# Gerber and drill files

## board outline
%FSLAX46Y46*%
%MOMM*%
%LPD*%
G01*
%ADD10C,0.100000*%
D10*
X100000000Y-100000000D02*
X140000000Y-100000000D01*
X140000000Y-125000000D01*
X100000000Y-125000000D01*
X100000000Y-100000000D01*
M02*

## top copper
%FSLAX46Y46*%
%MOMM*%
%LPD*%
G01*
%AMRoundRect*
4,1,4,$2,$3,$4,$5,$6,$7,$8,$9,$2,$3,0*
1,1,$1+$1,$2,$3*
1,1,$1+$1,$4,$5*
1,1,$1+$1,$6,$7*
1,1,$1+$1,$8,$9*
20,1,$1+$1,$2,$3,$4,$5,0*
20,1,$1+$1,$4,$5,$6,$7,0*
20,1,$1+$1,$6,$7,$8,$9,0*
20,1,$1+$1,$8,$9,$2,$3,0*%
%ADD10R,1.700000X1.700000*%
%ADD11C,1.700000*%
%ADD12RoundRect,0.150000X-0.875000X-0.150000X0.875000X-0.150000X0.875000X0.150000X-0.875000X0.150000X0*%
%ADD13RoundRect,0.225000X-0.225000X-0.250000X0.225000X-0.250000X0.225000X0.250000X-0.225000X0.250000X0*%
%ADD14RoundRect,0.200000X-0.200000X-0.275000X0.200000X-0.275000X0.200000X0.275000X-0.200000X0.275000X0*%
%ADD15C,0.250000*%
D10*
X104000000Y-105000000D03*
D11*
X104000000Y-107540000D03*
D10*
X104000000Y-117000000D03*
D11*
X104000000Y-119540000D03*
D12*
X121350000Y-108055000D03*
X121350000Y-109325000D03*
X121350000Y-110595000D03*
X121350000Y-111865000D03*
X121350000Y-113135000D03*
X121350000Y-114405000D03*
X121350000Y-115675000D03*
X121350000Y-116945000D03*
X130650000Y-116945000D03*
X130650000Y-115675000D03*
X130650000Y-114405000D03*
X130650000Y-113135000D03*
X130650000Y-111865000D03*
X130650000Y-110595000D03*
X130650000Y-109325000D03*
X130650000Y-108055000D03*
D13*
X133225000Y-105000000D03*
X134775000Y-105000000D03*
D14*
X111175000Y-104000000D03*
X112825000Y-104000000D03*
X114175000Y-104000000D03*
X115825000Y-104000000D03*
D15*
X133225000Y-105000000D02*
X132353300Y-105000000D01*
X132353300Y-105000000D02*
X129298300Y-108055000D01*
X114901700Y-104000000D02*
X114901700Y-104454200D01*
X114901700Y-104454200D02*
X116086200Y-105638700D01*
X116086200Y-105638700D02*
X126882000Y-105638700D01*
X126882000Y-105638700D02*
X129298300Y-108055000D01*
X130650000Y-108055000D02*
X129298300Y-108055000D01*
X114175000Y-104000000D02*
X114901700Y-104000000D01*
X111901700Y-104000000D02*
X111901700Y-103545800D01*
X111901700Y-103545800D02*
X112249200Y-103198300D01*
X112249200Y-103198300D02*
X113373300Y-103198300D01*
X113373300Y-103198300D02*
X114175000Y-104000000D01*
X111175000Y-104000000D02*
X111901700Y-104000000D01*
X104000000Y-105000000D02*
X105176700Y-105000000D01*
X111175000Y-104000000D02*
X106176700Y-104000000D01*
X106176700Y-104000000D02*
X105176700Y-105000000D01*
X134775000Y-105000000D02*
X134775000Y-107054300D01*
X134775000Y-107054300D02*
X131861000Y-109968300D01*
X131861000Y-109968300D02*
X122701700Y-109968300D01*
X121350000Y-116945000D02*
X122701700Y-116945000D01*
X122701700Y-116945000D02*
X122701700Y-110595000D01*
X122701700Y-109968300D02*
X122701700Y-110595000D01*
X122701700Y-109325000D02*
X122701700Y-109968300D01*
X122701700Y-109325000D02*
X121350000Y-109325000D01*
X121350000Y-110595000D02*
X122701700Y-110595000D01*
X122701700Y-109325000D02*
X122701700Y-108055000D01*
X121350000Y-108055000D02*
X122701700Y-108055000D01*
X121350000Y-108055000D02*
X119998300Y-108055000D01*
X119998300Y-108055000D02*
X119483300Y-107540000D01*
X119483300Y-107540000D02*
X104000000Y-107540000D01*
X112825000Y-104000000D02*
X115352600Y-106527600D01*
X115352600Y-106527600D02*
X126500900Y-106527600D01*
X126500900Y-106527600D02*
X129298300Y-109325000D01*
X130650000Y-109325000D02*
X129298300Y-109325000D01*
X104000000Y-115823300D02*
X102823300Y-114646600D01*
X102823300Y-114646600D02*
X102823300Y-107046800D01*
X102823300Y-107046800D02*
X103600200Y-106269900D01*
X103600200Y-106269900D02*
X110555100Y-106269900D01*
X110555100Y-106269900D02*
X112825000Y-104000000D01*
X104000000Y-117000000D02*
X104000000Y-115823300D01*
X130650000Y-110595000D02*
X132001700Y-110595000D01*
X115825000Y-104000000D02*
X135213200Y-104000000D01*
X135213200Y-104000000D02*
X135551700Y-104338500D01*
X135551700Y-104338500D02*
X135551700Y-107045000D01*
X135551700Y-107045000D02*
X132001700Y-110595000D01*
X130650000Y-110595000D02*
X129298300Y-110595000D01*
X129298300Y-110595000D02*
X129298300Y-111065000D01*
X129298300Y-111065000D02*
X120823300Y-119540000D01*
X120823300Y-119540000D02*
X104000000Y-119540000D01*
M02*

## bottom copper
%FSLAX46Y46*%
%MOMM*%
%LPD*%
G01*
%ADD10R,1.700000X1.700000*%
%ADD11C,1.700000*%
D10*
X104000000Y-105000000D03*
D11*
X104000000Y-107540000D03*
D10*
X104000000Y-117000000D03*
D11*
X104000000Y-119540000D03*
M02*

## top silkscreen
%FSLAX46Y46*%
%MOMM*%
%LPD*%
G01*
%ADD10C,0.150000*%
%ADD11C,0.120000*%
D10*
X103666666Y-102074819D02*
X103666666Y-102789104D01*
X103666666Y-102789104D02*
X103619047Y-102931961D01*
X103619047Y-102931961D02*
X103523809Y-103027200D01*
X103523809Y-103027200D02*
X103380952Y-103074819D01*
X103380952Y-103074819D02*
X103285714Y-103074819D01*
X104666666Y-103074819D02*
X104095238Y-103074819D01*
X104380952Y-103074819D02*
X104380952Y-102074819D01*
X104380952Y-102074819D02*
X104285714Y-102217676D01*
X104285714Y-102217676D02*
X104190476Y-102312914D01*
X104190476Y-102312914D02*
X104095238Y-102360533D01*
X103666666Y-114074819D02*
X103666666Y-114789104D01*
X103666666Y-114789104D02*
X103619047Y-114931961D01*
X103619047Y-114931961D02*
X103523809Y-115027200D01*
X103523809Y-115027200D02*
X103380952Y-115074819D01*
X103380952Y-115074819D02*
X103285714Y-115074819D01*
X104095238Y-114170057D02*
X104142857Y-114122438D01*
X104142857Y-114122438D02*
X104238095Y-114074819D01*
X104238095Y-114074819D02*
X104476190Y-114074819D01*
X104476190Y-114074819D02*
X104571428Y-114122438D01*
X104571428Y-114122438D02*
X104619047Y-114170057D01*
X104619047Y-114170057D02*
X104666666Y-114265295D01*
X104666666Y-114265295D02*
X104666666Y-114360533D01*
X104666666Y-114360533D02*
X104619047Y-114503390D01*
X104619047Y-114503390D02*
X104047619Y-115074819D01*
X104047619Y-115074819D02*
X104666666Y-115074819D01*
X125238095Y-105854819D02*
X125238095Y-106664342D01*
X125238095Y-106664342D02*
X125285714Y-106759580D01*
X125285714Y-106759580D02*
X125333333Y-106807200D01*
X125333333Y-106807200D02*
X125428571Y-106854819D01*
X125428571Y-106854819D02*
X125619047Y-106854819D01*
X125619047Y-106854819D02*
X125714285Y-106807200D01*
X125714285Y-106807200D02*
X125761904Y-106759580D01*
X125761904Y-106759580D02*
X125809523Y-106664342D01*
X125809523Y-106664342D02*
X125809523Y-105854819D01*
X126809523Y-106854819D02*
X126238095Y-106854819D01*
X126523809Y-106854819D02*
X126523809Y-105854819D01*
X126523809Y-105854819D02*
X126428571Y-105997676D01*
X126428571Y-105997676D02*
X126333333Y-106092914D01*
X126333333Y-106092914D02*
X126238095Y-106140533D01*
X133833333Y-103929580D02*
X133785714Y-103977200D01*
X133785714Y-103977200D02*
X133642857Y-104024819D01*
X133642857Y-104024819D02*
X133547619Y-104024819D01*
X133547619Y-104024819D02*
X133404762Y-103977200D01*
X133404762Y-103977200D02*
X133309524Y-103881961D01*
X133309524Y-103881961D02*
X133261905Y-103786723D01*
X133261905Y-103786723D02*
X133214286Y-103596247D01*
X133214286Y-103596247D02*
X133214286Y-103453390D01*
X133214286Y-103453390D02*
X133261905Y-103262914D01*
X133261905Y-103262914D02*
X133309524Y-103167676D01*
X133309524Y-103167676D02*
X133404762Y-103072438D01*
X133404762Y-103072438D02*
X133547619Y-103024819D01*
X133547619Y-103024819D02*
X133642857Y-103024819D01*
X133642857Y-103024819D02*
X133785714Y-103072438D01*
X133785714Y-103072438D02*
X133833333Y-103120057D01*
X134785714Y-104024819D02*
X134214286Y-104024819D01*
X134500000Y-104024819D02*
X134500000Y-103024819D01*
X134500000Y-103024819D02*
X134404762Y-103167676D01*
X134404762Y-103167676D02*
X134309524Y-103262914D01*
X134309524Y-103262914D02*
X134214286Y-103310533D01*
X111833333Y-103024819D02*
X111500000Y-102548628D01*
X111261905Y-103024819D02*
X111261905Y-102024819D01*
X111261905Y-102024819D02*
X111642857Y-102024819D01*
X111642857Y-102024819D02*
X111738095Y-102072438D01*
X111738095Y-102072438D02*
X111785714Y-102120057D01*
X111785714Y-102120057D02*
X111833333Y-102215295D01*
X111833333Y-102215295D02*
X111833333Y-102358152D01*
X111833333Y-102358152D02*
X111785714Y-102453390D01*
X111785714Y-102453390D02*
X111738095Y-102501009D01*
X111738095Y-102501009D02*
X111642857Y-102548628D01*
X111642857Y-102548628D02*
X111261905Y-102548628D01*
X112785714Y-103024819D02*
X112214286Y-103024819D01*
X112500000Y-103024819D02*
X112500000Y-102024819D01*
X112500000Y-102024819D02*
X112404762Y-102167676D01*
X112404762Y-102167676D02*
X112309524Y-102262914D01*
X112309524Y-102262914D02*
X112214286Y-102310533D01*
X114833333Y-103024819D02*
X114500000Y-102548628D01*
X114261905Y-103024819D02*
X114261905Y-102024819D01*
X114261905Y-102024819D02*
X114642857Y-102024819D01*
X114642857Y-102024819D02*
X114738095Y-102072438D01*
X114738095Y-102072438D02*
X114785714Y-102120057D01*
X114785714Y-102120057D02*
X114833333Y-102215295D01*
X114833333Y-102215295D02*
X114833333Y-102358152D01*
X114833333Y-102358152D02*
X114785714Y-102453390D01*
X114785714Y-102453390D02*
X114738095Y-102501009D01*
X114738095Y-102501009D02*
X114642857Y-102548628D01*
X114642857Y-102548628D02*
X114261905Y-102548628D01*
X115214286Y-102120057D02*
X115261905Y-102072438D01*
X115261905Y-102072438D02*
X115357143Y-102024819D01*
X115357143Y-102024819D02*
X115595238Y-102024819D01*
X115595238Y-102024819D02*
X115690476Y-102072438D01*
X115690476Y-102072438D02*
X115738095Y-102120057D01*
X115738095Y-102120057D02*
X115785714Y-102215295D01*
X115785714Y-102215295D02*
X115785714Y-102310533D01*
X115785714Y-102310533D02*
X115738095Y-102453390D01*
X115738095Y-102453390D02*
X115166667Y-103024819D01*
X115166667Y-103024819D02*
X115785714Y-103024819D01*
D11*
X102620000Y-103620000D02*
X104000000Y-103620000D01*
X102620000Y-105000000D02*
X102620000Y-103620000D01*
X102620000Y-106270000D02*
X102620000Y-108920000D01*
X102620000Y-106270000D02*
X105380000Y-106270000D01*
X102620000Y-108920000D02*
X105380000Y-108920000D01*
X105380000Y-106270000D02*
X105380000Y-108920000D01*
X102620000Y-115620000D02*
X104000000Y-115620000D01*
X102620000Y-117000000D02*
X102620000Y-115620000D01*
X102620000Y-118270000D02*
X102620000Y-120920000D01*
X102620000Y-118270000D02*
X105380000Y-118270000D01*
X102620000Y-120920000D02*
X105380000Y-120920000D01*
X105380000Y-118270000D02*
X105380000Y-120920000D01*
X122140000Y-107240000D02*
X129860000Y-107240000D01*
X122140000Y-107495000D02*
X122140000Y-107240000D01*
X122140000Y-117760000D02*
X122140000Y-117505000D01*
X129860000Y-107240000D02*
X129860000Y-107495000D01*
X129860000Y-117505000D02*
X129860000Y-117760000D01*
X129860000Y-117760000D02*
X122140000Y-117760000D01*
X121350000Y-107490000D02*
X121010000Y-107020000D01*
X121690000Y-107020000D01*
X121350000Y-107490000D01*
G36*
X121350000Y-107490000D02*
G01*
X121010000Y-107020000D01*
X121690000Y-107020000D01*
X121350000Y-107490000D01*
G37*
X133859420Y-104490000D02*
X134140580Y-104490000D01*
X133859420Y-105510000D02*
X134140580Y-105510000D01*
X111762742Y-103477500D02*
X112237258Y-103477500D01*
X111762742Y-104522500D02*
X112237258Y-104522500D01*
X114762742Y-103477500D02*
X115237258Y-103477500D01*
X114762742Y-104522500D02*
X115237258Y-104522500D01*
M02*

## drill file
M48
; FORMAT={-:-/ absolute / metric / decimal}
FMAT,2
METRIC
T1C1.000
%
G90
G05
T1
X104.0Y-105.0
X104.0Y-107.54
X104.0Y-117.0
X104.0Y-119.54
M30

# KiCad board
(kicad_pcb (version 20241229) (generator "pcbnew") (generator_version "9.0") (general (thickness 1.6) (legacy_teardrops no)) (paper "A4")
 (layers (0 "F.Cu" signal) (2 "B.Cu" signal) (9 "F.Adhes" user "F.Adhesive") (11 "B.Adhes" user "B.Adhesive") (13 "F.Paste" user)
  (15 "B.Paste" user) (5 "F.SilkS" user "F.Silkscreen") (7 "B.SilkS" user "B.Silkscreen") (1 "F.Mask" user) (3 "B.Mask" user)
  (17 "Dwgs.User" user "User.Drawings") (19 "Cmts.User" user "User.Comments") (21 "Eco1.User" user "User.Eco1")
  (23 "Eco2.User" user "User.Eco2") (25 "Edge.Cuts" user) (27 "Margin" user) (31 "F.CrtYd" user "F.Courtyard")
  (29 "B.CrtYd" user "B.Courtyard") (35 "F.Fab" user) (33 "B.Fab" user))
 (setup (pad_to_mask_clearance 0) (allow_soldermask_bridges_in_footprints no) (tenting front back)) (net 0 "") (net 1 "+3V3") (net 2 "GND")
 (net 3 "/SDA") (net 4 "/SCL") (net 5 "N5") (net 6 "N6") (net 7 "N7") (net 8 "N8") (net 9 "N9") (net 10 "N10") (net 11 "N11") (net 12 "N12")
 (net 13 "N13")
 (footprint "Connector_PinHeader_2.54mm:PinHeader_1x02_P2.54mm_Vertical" (layer "F.Cu") (at 104 105)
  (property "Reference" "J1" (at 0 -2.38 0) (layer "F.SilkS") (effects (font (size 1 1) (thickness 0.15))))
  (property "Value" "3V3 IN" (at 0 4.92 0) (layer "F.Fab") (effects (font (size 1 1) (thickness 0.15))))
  (fp_line (start -1.38 -1.38) (end 0 -1.38) (stroke (width 0.12) (type solid)) (layer "F.SilkS"))
  (fp_line (start -1.38 0) (end -1.38 -1.38) (stroke (width 0.12) (type solid)) (layer "F.SilkS"))
  (fp_line (start -1.38 1.27) (end -1.38 3.92) (stroke (width 0.12) (type solid)) (layer "F.SilkS"))
  (fp_line (start -1.38 1.27) (end 1.38 1.27) (stroke (width 0.12) (type solid)) (layer "F.SilkS"))
  (fp_line (start -1.38 3.92) (end 1.38 3.92) (stroke (width 0.12) (type solid)) (layer "F.SilkS"))
  (fp_line (start 1.38 1.27) (end 1.38 3.92) (stroke (width 0.12) (type solid)) (layer "F.SilkS"))
  (pad "1" thru_hole rect (at 0 0) (size 1.7 1.7) (drill 1) (layers "*.Cu" "*.Mask") (remove_unused_layers no) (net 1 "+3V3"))
  (pad "2" thru_hole circle (at 0 2.54) (size 1.7 1.7) (drill 1) (layers "*.Cu" "*.Mask") (remove_unused_layers no) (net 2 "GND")))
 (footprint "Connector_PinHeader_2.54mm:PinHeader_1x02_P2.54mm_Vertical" (layer "F.Cu") (at 104 117)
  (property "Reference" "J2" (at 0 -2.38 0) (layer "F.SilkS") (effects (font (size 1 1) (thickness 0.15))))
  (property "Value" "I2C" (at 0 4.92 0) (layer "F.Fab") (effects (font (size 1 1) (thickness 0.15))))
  (fp_line (start -1.38 -1.38) (end 0 -1.38) (stroke (width 0.12) (type solid)) (layer "F.SilkS"))
  (fp_line (start -1.38 0) (end -1.38 -1.38) (stroke (width 0.12) (type solid)) (layer "F.SilkS"))
  (fp_line (start -1.38 1.27) (end -1.38 3.92) (stroke (width 0.12) (type solid)) (layer "F.SilkS"))
  (fp_line (start -1.38 1.27) (end 1.38 1.27) (stroke (width 0.12) (type solid)) (layer "F.SilkS"))
  (fp_line (start -1.38 3.92) (end 1.38 3.92) (stroke (width 0.12) (type solid)) (layer "F.SilkS"))
  (fp_line (start 1.38 1.27) (end 1.38 3.92) (stroke (width 0.12) (type solid)) (layer "F.SilkS"))
  (pad "1" thru_hole rect (at 0 0) (size 1.7 1.7) (drill 1) (layers "*.Cu" "*.Mask") (remove_unused_layers no) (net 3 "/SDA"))
  (pad "2" thru_hole circle (at 0 2.54) (size 1.7 1.7) (drill 1) (layers "*.Cu" "*.Mask") (remove_unused_layers no) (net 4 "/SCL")))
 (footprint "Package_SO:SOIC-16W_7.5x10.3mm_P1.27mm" (layer "F.Cu") (at 126 112.5)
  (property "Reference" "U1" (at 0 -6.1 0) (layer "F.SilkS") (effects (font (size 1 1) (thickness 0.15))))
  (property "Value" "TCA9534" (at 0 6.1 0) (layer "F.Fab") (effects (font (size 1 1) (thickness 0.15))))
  (fp_line (start -3.86 -5.26) (end 3.86 -5.26) (stroke (width 0.12) (type solid)) (layer "F.SilkS"))
  (fp_line (start -3.86 -5.005) (end -3.86 -5.26) (stroke (width 0.12) (type solid)) (layer "F.SilkS"))
  (fp_line (start -3.86 5.26) (end -3.86 5.005) (stroke (width 0.12) (type solid)) (layer "F.SilkS"))
  (fp_line (start 3.86 -5.26) (end 3.86 -5.005) (stroke (width 0.12) (type solid)) (layer "F.SilkS"))
  (fp_line (start 3.86 5.005) (end 3.86 5.26) (stroke (width 0.12) (type solid)) (layer "F.SilkS"))
  (fp_line (start 3.86 5.26) (end -3.86 5.26) (stroke (width 0.12) (type solid)) (layer "F.SilkS"))
  (fp_poly (pts (xy -4.65 -5.01) (xy -4.99 -5.48) (xy -4.31 -5.48)) (stroke (width 0.12) (type solid)) (fill yes) (layer "F.SilkS"))
  (pad "1" smd roundrect (at -4.65 -4.445) (size 2.05 0.6) (layers "F.Cu" "F.Mask" "F.Paste") (roundrect_rratio 0.25) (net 2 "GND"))
  (pad "2" smd roundrect (at -4.65 -3.175) (size 2.05 0.6) (layers "F.Cu" "F.Mask" "F.Paste") (roundrect_rratio 0.25) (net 2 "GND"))
  (pad "3" smd roundrect (at -4.65 -1.905) (size 2.05 0.6) (layers "F.Cu" "F.Mask" "F.Paste") (roundrect_rratio 0.25) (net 2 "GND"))
  (pad "4" smd roundrect (at -4.65 -0.635) (size 2.05 0.6) (layers "F.Cu" "F.Mask" "F.Paste") (roundrect_rratio 0.25) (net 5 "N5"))
  (pad "5" smd roundrect (at -4.65 0.635) (size 2.05 0.6) (layers "F.Cu" "F.Mask" "F.Paste") (roundrect_rratio 0.25) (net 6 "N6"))
  (pad "6" smd roundrect (at -4.65 1.905) (size 2.05 0.6) (layers "F.Cu" "F.Mask" "F.Paste") (roundrect_rratio 0.25) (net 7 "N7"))
  (pad "7" smd roundrect (at -4.65 3.175) (size 2.05 0.6) (layers "F.Cu" "F.Mask" "F.Paste") (roundrect_rratio 0.25) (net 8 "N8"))
  (pad "8" smd roundrect (at -4.65 4.445) (size 2.05 0.6) (layers "F.Cu" "F.Mask" "F.Paste") (roundrect_rratio 0.25) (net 2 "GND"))
  (pad "9" smd roundrect (at 4.65 4.445) (size 2.05 0.6) (layers "F.Cu" "F.Mask" "F.Paste") (roundrect_rratio 0.25) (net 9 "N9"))
  (pad "10" smd roundrect (at 4.65 3.175) (size 2.05 0.6) (layers "F.Cu" "F.Mask" "F.Paste") (roundrect_rratio 0.25) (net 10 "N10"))
  (pad "11" smd roundrect (at 4.65 1.905) (size 2.05 0.6) (layers "F.Cu" "F.Mask" "F.Paste") (roundrect_rratio 0.25) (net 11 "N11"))
  (pad "12" smd roundrect (at 4.65 0.635) (size 2.05 0.6) (layers "F.Cu" "F.Mask" "F.Paste") (roundrect_rratio 0.25) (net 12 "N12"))
  (pad "13" smd roundrect (at 4.65 -0.635) (size 2.05 0.6) (layers "F.Cu" "F.Mask" "F.Paste") (roundrect_rratio 0.25) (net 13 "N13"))
  (pad "14" smd roundrect (at 4.65 -1.905) (size 2.05 0.6) (layers "F.Cu" "F.Mask" "F.Paste") (roundrect_rratio 0.25) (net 4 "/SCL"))
  (pad "15" smd roundrect (at 4.65 -3.175) (size 2.05 0.6) (layers "F.Cu" "F.Mask" "F.Paste") (roundrect_rratio 0.25) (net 3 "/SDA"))
  (pad "16" smd roundrect (at 4.65 -4.445) (size 2.05 0.6) (layers "F.Cu" "F.Mask" "F.Paste") (roundrect_rratio 0.25) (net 1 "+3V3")))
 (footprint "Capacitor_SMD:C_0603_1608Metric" (layer "F.Cu") (at 134 105)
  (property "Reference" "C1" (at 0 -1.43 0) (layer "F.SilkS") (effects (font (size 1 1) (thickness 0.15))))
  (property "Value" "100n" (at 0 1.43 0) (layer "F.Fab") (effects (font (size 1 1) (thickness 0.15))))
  (fp_line (start -0.14058 -0.51) (end 0.14058 -0.51) (stroke (width 0.12) (type solid)) (layer "F.SilkS"))
  (fp_line (start -0.14058 0.51) (end 0.14058 0.51) (stroke (width 0.12) (type solid)) (layer "F.SilkS"))
  (pad "1" smd roundrect (at -0.775 0) (size 0.9 0.95) (layers "F.Cu" "F.Mask" "F.Paste") (roundrect_rratio 0.25) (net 1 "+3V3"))
  (pad "2" smd roundrect (at 0.775 0) (size 0.9 0.95) (layers "F.Cu" "F.Mask" "F.Paste") (roundrect_rratio 0.25) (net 2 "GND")))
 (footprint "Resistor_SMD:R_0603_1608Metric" (layer "F.Cu") (at 112 104)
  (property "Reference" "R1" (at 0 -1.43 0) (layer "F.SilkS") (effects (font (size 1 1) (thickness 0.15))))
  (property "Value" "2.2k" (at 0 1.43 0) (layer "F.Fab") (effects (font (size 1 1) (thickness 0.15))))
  (fp_line (start -0.237258 -0.5225) (end 0.237258 -0.5225) (stroke (width 0.12) (type solid)) (layer "F.SilkS"))
  (fp_line (start -0.237258 0.5225) (end 0.237258 0.5225) (stroke (width 0.12) (type solid)) (layer "F.SilkS"))
  (pad "1" smd roundrect (at -0.825 0) (size 0.8 0.95) (layers "F.Cu" "F.Mask" "F.Paste") (roundrect_rratio 0.25) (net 1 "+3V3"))
  (pad "2" smd roundrect (at 0.825 0) (size 0.8 0.95) (layers "F.Cu" "F.Mask" "F.Paste") (roundrect_rratio 0.25) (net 3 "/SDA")))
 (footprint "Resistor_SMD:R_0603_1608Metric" (layer "F.Cu") (at 115 104)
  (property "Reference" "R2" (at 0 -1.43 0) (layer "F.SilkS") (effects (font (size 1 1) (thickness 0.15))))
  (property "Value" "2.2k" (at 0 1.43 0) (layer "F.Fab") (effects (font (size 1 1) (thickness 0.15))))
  (fp_line (start -0.237258 -0.5225) (end 0.237258 -0.5225) (stroke (width 0.12) (type solid)) (layer "F.SilkS"))
  (fp_line (start -0.237258 0.5225) (end 0.237258 0.5225) (stroke (width 0.12) (type solid)) (layer "F.SilkS"))
  (pad "1" smd roundrect (at -0.825 0) (size 0.8 0.95) (layers "F.Cu" "F.Mask" "F.Paste") (roundrect_rratio 0.25) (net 1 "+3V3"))
  (pad "2" smd roundrect (at 0.825 0) (size 0.8 0.95) (layers "F.Cu" "F.Mask" "F.Paste") (roundrect_rratio 0.25) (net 4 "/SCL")))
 (gr_rect (start 100 100) (end 140 125) (stroke (width 0.1) (type default)) (fill no) (layer "Edge.Cuts"))
 (segment (start 133.225 105) (end 132.3533 105) (width 0.25) (layer "F.Cu") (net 1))
 (segment (start 132.3533 105) (end 129.2983 108.055) (width 0.25) (layer "F.Cu") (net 1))
 (segment (start 114.9017 104) (end 114.9017 104.4542) (width 0.25) (layer "F.Cu") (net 1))
 (segment (start 114.9017 104.4542) (end 116.0862 105.6387) (width 0.25) (layer "F.Cu") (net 1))
 (segment (start 116.0862 105.6387) (end 126.882 105.6387) (width 0.25) (layer "F.Cu") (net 1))
 (segment (start 126.882 105.6387) (end 129.2983 108.055) (width 0.25) (layer "F.Cu") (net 1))
 (segment (start 130.65 108.055) (end 129.2983 108.055) (width 0.25) (layer "F.Cu") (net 1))
 (segment (start 114.175 104) (end 114.9017 104) (width 0.25) (layer "F.Cu") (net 1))
 (segment (start 111.9017 104) (end 111.9017 103.5458) (width 0.25) (layer "F.Cu") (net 1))
 (segment (start 111.9017 103.5458) (end 112.2492 103.1983) (width 0.25) (layer "F.Cu") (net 1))
 (segment (start 112.2492 103.1983) (end 113.3733 103.1983) (width 0.25) (layer "F.Cu") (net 1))
 (segment (start 113.3733 103.1983) (end 114.175 104) (width 0.25) (layer "F.Cu") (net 1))
 (segment (start 111.175 104) (end 111.9017 104) (width 0.25) (layer "F.Cu") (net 1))
 (segment (start 104 105) (end 105.1767 105) (width 0.25) (layer "F.Cu") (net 1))
 (segment (start 111.175 104) (end 106.1767 104) (width 0.25) (layer "F.Cu") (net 1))
 (segment (start 106.1767 104) (end 105.1767 105) (width 0.25) (layer "F.Cu") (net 1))
 (segment (start 134.775 105) (end 134.775 107.0543) (width 0.25) (layer "F.Cu") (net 2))
 (segment (start 134.775 107.0543) (end 131.861 109.9683) (width 0.25) (layer "F.Cu") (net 2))
 (segment (start 131.861 109.9683) (end 122.7017 109.9683) (width 0.25) (layer "F.Cu") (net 2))
 (segment (start 121.35 116.945) (end 122.7017 116.945) (width 0.25) (layer "F.Cu") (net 2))
 (segment (start 122.7017 116.945) (end 122.7017 110.595) (width 0.25) (layer "F.Cu") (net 2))
 (segment (start 122.7017 109.9683) (end 122.7017 110.595) (width 0.25) (layer "F.Cu") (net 2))
 (segment (start 122.7017 109.325) (end 122.7017 109.9683) (width 0.25) (layer "F.Cu") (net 2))
 (segment (start 122.7017 109.325) (end 121.35 109.325) (width 0.25) (layer "F.Cu") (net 2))
 (segment (start 121.35 110.595) (end 122.7017 110.595) (width 0.25) (layer "F.Cu") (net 2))
 (segment (start 122.7017 109.325) (end 122.7017 108.055) (width 0.25) (layer "F.Cu") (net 2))
 (segment (start 121.35 108.055) (end 122.7017 108.055) (width 0.25) (layer "F.Cu") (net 2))
 (segment (start 121.35 108.055) (end 119.9983 108.055) (width 0.25) (layer "F.Cu") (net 2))
 (segment (start 119.9983 108.055) (end 119.4833 107.54) (width 0.25) (layer "F.Cu") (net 2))
 (segment (start 119.4833 107.54) (end 104 107.54) (width 0.25) (layer "F.Cu") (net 2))
 (segment (start 112.825 104) (end 115.3526 106.5276) (width 0.25) (layer "F.Cu") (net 3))
 (segment (start 115.3526 106.5276) (end 126.5009 106.5276) (width 0.25) (layer "F.Cu") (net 3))
 (segment (start 126.5009 106.5276) (end 129.2983 109.325) (width 0.25) (layer "F.Cu") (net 3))
 (segment (start 130.65 109.325) (end 129.2983 109.325) (width 0.25) (layer "F.Cu") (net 3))
 (segment (start 104 115.8233) (end 102.8233 114.6466) (width 0.25) (layer "F.Cu") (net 3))
 (segment (start 102.8233 114.6466) (end 102.8233 107.0468) (width 0.25) (layer "F.Cu") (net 3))
 (segment (start 102.8233 107.0468) (end 103.6002 106.2699) (width 0.25) (layer "F.Cu") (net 3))
 (segment (start 103.6002 106.2699) (end 110.5551 106.2699) (width 0.25) (layer "F.Cu") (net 3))
 (segment (start 110.5551 106.2699) (end 112.825 104) (width 0.25) (layer "F.Cu") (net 3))
 (segment (start 104 117) (end 104 115.8233) (width 0.25) (layer "F.Cu") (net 3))
 (segment (start 130.65 110.595) (end 132.0017 110.595) (width 0.25) (layer "F.Cu") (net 4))
 (segment (start 115.825 104) (end 135.2132 104) (width 0.25) (layer "F.Cu") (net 4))
 (segment (start 135.2132 104) (end 135.5517 104.3385) (width 0.25) (layer "F.Cu") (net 4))
 (segment (start 135.5517 104.3385) (end 135.5517 107.045) (width 0.25) (layer "F.Cu") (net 4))
 (segment (start 135.5517 107.045) (end 132.0017 110.595) (width 0.25) (layer "F.Cu") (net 4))
 (segment (start 130.65 110.595) (end 129.2983 110.595) (width 0.25) (layer "F.Cu") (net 4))
 (segment (start 129.2983 110.595) (end 129.2983 111.065) (width 0.25) (layer "F.Cu") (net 4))
 (segment (start 129.2983 111.065) (end 120.8233 119.54) (width 0.25) (layer "F.Cu") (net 4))
 (segment (start 120.8233 119.54) (end 104 119.54) (width 0.25) (layer "F.Cu") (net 4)))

